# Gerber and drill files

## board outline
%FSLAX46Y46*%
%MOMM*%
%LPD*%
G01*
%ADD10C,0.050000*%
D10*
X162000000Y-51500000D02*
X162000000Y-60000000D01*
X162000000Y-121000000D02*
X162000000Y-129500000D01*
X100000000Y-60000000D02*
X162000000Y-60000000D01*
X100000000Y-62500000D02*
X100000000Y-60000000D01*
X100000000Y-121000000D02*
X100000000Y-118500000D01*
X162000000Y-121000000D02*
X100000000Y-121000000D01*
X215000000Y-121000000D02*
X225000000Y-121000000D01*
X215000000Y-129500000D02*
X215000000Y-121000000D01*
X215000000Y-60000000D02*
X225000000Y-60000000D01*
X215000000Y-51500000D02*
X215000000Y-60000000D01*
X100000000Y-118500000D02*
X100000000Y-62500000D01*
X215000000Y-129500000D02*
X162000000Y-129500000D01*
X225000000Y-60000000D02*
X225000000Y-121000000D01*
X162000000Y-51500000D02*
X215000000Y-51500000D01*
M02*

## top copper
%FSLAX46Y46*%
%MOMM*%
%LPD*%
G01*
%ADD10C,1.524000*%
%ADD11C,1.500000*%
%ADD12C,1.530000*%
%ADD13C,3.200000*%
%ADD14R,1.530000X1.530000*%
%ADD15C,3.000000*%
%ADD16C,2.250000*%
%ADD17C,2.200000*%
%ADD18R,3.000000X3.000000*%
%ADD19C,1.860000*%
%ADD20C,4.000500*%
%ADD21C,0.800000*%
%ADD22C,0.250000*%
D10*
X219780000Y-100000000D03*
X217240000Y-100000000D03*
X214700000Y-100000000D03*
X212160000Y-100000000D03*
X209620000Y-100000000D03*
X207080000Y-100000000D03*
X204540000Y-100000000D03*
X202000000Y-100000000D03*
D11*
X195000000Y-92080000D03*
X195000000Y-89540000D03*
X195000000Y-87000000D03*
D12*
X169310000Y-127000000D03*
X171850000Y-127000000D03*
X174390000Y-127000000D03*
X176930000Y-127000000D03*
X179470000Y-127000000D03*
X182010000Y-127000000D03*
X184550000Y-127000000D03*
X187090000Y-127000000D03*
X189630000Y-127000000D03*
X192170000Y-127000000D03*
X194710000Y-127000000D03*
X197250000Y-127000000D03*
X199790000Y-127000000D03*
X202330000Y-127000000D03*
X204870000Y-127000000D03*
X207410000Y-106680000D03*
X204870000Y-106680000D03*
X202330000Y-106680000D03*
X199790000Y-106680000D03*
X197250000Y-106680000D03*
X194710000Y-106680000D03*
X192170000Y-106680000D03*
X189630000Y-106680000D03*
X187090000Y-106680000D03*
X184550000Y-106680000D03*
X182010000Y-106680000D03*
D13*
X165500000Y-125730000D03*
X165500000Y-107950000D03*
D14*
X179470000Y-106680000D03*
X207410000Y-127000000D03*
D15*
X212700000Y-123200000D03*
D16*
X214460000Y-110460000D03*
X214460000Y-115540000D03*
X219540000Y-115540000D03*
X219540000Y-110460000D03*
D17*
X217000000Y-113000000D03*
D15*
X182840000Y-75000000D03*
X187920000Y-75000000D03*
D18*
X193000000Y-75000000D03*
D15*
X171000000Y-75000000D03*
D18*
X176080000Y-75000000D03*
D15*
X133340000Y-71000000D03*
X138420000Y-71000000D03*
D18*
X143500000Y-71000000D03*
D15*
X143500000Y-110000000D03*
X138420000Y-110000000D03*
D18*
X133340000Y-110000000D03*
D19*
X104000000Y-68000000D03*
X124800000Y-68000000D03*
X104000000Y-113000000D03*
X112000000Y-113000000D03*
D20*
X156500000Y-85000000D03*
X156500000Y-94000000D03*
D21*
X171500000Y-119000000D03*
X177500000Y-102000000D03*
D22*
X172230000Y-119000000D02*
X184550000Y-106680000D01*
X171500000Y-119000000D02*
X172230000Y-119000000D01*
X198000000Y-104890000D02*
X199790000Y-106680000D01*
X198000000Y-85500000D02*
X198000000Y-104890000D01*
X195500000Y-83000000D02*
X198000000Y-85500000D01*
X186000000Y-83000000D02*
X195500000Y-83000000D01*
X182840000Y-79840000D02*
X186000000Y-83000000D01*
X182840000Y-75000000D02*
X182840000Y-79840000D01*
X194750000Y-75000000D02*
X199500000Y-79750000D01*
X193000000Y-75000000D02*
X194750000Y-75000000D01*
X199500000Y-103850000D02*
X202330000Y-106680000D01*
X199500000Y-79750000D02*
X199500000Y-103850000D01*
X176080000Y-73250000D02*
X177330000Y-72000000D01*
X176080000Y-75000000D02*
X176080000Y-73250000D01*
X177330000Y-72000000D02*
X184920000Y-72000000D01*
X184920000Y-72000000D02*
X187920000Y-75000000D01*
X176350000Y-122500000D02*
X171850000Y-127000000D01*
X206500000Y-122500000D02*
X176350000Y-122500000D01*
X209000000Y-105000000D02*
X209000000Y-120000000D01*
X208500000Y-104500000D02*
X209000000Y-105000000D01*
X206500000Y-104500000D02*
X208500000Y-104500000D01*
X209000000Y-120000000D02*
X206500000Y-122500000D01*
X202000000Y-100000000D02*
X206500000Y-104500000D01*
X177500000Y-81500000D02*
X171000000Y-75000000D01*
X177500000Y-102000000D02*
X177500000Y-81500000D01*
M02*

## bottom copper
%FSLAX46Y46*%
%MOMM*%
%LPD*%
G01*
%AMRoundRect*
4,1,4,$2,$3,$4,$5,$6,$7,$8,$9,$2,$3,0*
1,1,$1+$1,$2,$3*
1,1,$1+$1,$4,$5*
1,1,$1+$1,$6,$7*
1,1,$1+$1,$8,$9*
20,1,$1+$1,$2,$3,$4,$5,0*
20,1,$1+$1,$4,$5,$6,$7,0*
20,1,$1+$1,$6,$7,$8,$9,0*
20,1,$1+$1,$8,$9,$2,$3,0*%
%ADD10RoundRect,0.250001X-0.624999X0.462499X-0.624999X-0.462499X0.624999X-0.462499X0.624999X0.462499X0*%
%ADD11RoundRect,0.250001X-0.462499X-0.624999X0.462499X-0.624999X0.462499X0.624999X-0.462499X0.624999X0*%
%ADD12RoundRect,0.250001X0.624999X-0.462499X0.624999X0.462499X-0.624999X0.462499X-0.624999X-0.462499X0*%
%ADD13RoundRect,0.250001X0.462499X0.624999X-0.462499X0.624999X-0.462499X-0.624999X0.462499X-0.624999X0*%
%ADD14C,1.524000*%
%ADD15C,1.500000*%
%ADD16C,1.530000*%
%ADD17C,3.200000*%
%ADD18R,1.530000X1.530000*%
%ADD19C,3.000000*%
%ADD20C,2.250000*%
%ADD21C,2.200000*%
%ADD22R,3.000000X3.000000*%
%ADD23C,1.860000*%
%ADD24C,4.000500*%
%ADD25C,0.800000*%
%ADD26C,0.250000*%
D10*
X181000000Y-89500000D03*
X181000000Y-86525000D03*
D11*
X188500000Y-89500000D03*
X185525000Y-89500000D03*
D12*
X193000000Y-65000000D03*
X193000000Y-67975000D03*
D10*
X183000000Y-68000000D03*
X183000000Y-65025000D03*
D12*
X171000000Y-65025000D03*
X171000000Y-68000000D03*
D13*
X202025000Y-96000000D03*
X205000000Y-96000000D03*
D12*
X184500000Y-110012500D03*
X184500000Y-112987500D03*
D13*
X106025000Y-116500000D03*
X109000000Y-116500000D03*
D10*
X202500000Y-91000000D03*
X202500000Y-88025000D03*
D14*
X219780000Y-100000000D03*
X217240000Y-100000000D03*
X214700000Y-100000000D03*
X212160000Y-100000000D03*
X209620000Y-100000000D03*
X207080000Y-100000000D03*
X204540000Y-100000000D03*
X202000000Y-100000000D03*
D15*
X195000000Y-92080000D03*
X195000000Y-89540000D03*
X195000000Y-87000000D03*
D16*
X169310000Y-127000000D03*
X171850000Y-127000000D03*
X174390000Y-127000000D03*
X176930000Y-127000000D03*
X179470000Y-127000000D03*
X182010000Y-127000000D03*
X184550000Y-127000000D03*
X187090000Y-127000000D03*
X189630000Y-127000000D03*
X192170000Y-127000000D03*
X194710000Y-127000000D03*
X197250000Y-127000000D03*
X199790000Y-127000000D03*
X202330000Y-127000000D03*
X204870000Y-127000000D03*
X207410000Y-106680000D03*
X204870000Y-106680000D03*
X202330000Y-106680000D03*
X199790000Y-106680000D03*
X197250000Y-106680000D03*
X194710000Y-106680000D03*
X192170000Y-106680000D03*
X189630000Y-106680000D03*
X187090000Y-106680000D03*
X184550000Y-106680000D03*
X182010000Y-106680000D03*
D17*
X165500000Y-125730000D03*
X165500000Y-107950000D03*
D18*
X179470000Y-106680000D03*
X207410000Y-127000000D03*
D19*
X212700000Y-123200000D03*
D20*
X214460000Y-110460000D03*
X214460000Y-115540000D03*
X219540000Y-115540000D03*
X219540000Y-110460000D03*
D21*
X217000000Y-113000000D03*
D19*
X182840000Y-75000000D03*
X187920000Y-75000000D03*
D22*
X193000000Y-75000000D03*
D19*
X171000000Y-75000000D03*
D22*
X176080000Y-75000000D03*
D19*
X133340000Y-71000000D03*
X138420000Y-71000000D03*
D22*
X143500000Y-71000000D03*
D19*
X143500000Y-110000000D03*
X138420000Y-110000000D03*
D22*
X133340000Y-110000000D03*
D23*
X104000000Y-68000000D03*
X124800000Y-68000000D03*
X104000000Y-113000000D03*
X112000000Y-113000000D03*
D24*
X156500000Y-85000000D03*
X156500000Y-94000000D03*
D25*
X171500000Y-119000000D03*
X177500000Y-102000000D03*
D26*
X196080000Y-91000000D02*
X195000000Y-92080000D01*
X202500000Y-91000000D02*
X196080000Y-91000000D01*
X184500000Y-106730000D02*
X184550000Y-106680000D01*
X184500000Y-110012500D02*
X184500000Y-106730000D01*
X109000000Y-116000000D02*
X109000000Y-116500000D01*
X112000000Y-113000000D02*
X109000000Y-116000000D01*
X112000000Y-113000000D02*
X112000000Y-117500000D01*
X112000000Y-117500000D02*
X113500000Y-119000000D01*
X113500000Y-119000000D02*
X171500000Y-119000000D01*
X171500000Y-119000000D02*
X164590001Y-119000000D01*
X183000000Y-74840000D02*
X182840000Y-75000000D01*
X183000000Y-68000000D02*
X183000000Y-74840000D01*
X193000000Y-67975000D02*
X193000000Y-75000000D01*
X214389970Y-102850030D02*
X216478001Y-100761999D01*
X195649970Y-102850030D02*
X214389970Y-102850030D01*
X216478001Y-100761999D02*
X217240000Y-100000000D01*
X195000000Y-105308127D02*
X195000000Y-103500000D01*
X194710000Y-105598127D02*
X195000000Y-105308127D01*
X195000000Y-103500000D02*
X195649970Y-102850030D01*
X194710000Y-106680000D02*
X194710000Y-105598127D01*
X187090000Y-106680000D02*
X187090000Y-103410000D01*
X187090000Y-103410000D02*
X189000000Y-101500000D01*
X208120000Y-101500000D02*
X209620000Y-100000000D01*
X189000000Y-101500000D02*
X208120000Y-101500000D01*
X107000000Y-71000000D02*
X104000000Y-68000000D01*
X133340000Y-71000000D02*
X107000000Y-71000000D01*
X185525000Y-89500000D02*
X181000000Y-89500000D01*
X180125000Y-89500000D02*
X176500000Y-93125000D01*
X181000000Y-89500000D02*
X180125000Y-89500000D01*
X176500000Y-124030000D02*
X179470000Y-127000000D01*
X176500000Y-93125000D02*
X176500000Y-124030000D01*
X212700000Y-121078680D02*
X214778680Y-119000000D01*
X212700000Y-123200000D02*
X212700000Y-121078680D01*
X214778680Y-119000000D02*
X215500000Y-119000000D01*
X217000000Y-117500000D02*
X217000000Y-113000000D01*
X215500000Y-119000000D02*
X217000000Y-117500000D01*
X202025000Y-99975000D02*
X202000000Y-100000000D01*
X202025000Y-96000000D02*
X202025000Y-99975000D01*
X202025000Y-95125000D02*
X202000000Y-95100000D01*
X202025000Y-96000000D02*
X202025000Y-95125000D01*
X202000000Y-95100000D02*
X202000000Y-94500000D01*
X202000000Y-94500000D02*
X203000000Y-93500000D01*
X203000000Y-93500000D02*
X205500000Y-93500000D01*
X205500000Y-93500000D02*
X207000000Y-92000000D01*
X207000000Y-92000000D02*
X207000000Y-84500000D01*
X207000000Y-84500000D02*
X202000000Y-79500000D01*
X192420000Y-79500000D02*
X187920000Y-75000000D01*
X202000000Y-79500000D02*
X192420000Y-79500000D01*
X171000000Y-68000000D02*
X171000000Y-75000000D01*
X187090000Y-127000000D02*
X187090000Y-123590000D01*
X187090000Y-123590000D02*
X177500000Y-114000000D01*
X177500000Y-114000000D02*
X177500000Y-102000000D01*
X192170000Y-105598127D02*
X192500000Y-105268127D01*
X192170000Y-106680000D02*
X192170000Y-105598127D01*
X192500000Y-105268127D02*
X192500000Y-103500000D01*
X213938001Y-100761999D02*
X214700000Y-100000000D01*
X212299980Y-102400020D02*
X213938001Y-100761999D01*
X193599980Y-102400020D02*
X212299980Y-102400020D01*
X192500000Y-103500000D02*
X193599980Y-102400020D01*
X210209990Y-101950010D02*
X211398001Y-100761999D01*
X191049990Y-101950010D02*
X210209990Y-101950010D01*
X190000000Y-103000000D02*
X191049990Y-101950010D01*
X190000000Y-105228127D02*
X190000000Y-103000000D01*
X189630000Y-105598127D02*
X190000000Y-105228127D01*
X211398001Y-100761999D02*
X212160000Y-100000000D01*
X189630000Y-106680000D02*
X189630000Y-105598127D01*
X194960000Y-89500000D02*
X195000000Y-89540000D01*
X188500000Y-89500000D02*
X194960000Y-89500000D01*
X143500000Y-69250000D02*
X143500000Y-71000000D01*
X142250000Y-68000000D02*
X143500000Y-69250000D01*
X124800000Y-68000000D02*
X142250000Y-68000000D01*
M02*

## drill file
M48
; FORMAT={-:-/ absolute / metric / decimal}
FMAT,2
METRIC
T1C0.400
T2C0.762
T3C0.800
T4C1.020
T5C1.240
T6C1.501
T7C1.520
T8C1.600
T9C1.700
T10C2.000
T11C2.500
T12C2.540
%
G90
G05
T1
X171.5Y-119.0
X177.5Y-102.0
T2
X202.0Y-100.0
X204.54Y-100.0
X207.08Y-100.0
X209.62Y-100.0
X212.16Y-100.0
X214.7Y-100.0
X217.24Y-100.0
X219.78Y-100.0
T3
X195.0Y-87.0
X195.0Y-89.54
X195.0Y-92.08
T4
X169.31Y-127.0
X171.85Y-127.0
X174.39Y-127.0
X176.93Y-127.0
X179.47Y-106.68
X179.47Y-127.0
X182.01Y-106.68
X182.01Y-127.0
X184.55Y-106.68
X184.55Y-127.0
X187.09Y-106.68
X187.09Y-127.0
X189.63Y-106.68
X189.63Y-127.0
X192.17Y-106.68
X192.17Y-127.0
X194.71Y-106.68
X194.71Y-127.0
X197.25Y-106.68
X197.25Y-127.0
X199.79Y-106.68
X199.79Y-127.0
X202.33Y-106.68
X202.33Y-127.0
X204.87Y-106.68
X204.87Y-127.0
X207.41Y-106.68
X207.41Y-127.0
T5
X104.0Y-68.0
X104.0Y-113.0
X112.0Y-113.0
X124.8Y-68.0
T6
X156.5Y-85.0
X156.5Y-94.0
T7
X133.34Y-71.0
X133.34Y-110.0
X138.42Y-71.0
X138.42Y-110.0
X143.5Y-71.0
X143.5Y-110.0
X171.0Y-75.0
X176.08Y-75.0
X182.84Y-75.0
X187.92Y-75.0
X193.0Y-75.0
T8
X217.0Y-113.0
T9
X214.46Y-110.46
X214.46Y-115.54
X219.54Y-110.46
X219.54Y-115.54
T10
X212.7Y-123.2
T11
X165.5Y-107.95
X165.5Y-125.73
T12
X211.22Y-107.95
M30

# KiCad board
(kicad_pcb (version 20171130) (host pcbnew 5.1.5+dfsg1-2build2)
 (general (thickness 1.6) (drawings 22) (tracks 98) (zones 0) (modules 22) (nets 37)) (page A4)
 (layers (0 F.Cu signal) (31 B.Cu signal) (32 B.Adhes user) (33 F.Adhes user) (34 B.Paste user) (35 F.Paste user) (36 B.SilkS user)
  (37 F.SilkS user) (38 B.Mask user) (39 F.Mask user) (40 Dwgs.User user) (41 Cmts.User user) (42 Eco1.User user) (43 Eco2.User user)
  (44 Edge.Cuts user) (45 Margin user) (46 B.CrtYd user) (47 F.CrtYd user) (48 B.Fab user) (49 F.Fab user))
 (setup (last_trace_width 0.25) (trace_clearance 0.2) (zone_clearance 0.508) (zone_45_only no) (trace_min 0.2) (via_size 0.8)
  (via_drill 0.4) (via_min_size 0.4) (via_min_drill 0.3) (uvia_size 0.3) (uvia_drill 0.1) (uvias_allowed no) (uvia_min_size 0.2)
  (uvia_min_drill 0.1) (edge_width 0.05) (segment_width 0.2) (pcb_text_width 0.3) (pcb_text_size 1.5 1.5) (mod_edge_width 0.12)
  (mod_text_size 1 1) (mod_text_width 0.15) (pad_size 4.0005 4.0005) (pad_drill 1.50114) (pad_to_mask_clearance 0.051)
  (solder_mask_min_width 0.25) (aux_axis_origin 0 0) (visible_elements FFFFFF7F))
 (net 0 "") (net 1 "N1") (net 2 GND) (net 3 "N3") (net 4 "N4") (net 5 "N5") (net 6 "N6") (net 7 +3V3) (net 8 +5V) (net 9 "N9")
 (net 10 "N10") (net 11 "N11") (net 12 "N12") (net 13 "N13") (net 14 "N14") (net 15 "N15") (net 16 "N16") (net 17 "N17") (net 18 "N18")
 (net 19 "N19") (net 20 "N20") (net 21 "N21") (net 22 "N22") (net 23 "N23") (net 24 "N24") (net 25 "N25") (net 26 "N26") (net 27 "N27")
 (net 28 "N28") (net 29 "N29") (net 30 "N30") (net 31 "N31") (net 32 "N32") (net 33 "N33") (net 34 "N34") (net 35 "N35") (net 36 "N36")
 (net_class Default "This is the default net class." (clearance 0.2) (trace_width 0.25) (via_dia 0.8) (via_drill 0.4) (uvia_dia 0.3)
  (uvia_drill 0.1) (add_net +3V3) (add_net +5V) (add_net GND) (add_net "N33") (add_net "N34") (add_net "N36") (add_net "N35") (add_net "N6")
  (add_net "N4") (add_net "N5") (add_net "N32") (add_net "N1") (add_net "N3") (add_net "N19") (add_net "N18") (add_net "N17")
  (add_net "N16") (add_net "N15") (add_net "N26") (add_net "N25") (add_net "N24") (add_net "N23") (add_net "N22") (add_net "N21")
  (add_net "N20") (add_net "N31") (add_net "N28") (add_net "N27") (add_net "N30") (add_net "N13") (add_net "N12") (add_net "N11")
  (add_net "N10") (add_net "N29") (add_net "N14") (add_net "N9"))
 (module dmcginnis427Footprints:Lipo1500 (layer F.Cu) (at 150.5 105.5 90)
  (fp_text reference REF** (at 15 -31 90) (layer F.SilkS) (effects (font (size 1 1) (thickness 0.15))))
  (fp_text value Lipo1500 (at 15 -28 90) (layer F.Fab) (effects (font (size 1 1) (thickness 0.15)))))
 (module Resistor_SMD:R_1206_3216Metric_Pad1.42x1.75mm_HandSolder (layer B.Cu) (at 181 88.0125 270)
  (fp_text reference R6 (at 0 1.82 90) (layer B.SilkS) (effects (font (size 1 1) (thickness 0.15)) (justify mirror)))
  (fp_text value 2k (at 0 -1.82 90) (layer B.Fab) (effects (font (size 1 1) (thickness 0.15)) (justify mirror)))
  (pad 2 smd roundrect (at 1.4875 0 270) (size 1.425 1.75) (layers B.Cu B.Paste B.Mask) (roundrect_rratio 0.175439) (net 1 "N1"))
  (pad 1 smd roundrect (at -1.4875 0 270) (size 1.425 1.75) (layers B.Cu B.Paste B.Mask) (roundrect_rratio 0.175439) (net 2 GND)))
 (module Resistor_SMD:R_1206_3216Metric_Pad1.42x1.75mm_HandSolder (layer B.Cu) (at 187.0125 89.5)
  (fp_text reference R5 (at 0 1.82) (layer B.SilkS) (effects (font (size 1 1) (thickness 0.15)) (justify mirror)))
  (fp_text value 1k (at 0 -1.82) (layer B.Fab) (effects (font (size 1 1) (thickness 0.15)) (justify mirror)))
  (pad 2 smd roundrect (at 1.4875 0) (size 1.425 1.75) (layers B.Cu B.Paste B.Mask) (roundrect_rratio 0.175439) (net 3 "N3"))
  (pad 1 smd roundrect (at -1.4875 0) (size 1.425 1.75) (layers B.Cu B.Paste B.Mask) (roundrect_rratio 0.175439) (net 1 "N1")))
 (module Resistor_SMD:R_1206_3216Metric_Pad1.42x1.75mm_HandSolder (layer B.Cu) (at 193 66.4875 90)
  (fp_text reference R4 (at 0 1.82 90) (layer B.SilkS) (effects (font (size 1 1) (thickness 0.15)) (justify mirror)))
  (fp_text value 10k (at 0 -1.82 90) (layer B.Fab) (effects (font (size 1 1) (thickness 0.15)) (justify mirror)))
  (pad 2 smd roundrect (at 1.4875 0 90) (size 1.425 1.75) (layers B.Cu B.Paste B.Mask) (roundrect_rratio 0.175439) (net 2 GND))
  (pad 1 smd roundrect (at -1.4875 0 90) (size 1.425 1.75) (layers B.Cu B.Paste B.Mask) (roundrect_rratio 0.175439) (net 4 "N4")))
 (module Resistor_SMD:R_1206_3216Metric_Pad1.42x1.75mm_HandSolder (layer B.Cu) (at 183 66.5125 270)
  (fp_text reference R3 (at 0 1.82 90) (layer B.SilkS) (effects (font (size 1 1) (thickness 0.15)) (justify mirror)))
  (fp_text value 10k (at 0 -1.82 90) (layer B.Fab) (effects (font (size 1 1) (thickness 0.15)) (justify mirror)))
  (pad 2 smd roundrect (at 1.4875 0 270) (size 1.425 1.75) (layers B.Cu B.Paste B.Mask) (roundrect_rratio 0.175439) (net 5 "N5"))
  (pad 1 smd roundrect (at -1.4875 0 270) (size 1.425 1.75) (layers B.Cu B.Paste B.Mask) (roundrect_rratio 0.175439) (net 2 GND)))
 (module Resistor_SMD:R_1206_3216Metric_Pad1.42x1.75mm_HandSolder (layer B.Cu) (at 171 66.5125 90)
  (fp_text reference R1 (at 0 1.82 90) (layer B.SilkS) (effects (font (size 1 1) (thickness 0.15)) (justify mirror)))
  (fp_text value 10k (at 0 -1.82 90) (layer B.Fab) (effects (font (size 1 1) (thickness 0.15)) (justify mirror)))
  (pad 2 smd roundrect (at 1.4875 0 90) (size 1.425 1.75) (layers B.Cu B.Paste B.Mask) (roundrect_rratio 0.175439) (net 2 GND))
  (pad 1 smd roundrect (at -1.4875 0 90) (size 1.425 1.75) (layers B.Cu B.Paste B.Mask) (roundrect_rratio 0.175439) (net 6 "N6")))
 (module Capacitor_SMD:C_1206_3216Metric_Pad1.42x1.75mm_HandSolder (layer B.Cu) (at 203.5125 96 180)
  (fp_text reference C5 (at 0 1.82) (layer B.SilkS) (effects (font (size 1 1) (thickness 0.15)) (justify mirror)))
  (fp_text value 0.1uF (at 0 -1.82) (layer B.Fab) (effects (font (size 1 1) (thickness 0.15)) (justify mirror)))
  (pad 2 smd roundrect (at 1.4875 0 180) (size 1.425 1.75) (layers B.Cu B.Paste B.Mask) (roundrect_rratio 0.175439) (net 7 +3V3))
  (pad 1 smd roundrect (at -1.4875 0 180) (size 1.425 1.75) (layers B.Cu B.Paste B.Mask) (roundrect_rratio 0.175439) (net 2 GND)))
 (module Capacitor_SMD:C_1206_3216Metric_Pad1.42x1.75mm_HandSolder (layer B.Cu) (at 184.5 111.5 90)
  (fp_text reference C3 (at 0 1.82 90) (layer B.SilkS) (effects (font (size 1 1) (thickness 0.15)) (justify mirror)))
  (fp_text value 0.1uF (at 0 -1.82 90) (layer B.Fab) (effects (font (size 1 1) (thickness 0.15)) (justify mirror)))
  (pad 2 smd roundrect (at 1.4875 0 90) (size 1.425 1.75) (layers B.Cu B.Paste B.Mask) (roundrect_rratio 0.175439) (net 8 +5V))
  (pad 1 smd roundrect (at -1.4875 0 90) (size 1.425 1.75) (layers B.Cu B.Paste B.Mask) (roundrect_rratio 0.175439) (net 2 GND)))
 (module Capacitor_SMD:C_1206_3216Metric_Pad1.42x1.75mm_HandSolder (layer B.Cu) (at 107.5125 116.5 180)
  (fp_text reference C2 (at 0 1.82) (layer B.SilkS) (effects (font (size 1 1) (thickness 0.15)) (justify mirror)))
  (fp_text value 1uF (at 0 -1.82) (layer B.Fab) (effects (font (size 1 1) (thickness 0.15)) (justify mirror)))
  (pad 2 smd roundrect (at 1.4875 0 180) (size 1.425 1.75) (layers B.Cu B.Paste B.Mask) (roundrect_rratio 0.175439) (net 2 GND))
  (pad 1 smd roundrect (at -1.4875 0 180) (size 1.425 1.75) (layers B.Cu B.Paste B.Mask) (roundrect_rratio 0.175439) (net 8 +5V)))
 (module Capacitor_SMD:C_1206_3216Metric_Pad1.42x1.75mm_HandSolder (layer B.Cu) (at 202.5 89.5125 270)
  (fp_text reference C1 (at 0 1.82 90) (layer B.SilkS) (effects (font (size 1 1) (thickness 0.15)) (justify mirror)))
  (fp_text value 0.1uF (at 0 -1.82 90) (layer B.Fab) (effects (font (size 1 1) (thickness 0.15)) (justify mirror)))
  (pad 2 smd roundrect (at 1.4875 0 270) (size 1.425 1.75) (layers B.Cu B.Paste B.Mask) (roundrect_rratio 0.175439) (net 8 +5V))
  (pad 1 smd roundrect (at -1.4875 0 270) (size 1.425 1.75) (layers B.Cu B.Paste B.Mask) (roundrect_rratio 0.175439) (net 2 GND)))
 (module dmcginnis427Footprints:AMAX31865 (layer F.Cu) (at 202 100)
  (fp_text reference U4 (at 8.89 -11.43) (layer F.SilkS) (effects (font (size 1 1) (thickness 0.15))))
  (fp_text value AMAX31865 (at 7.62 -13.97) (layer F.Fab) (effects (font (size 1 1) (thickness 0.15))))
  (pad 8 thru_hole circle (at 17.78 0) (size 1.524 1.524) (drill 0.762) (layers *.Cu *.Mask) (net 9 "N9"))
  (pad 7 thru_hole circle (at 15.24 0) (size 1.524 1.524) (drill 0.762) (layers *.Cu *.Mask) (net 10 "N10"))
  (pad 6 thru_hole circle (at 12.7 0) (size 1.524 1.524) (drill 0.762) (layers *.Cu *.Mask) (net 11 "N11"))
  (pad 5 thru_hole circle (at 10.16 0) (size 1.524 1.524) (drill 0.762) (layers *.Cu *.Mask) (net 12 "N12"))
  (pad 4 thru_hole circle (at 7.62 0) (size 1.524 1.524) (drill 0.762) (layers *.Cu *.Mask) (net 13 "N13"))
  (pad 3 thru_hole circle (at 5.08 0) (size 1.524 1.524) (drill 0.762) (layers *.Cu *.Mask) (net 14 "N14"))
  (pad 2 thru_hole circle (at 2.54 0) (size 1.524 1.524) (drill 0.762) (layers *.Cu *.Mask) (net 2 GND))
  (pad 1 thru_hole circle (at 0 0) (size 1.524 1.524) (drill 0.762) (layers *.Cu *.Mask) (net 7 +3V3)))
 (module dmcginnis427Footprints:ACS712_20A (layer F.Cu) (at 195 89.54 270)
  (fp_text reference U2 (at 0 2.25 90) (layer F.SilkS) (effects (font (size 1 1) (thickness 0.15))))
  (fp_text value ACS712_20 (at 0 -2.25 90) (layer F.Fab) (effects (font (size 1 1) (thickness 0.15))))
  (pad 3 thru_hole circle (at 2.54 0 270) (size 1.5 1.5) (drill 0.8) (layers *.Cu *.Mask) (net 8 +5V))
  (pad 2 thru_hole circle (at 0 0 270) (size 1.5 1.5) (drill 0.8) (layers *.Cu *.Mask) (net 3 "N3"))
  (pad 1 thru_hole circle (at -2.54 0 270) (size 1.5 1.5) (drill 0.8) (layers *.Cu *.Mask) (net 2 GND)))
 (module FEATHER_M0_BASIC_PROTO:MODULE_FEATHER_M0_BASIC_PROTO (layer F.Cu) (at 188.36 116.84)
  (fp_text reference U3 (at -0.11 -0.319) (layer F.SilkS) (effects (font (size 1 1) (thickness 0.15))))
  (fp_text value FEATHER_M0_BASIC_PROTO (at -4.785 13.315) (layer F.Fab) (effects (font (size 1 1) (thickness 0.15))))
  (pad P1_16 thru_hole circle (at -19.05 10.16) (size 1.53 1.53) (drill 1.02) (layers *.Cu *.Mask) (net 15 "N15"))
  (pad P1_15 thru_hole circle (at -16.51 10.16) (size 1.53 1.53) (drill 1.02) (layers *.Cu *.Mask) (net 7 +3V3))
  (pad P1_14 thru_hole circle (at -13.97 10.16) (size 1.53 1.53) (drill 1.02) (layers *.Cu *.Mask) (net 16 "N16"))
  (pad P1_13 thru_hole circle (at -11.43 10.16) (size 1.53 1.53) (drill 1.02) (layers *.Cu *.Mask) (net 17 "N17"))
  (pad P1_12 thru_hole circle (at -8.89 10.16) (size 1.53 1.53) (drill 1.02) (layers *.Cu *.Mask) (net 1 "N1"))
  (pad P1_11 thru_hole circle (at -6.35 10.16) (size 1.53 1.53) (drill 1.02) (layers *.Cu *.Mask) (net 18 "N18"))
  (pad P1_10 thru_hole circle (at -3.81 10.16) (size 1.53 1.53) (drill 1.02) (layers *.Cu *.Mask) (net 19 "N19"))
  (pad P1_9 thru_hole circle (at -1.27 10.16) (size 1.53 1.53) (drill 1.02) (layers *.Cu *.Mask) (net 6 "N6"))
  (pad P1_8 thru_hole circle (at 1.27 10.16) (size 1.53 1.53) (drill 1.02) (layers *.Cu *.Mask) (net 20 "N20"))
  (pad P1_7 thru_hole circle (at 3.81 10.16) (size 1.53 1.53) (drill 1.02) (layers *.Cu *.Mask) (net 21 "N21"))
  (pad P1_6 thru_hole circle (at 6.35 10.16) (size 1.53 1.53) (drill 1.02) (layers *.Cu *.Mask) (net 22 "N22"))
  (pad P1_5 thru_hole circle (at 8.89 10.16) (size 1.53 1.53) (drill 1.02) (layers *.Cu *.Mask) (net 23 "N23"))
  (pad P1_4 thru_hole circle (at 11.43 10.16) (size 1.53 1.53) (drill 1.02) (layers *.Cu *.Mask) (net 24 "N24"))
  (pad P1_3 thru_hole circle (at 13.97 10.16) (size 1.53 1.53) (drill 1.02) (layers *.Cu *.Mask) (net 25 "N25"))
  (pad P1_2 thru_hole circle (at 16.51 10.16) (size 1.53 1.53) (drill 1.02) (layers *.Cu *.Mask) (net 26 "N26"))
  (pad P2_12 thru_hole circle (at 19.05 -10.16) (size 1.53 1.53) (drill 1.02) (layers *.Cu *.Mask) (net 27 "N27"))
  (pad P2_11 thru_hole circle (at 16.51 -10.16) (size 1.53 1.53) (drill 1.02) (layers *.Cu *.Mask) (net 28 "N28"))
  (pad P2_10 thru_hole circle (at 13.97 -10.16) (size 1.53 1.53) (drill 1.02) (layers *.Cu *.Mask) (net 4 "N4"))
  (pad P2_9 thru_hole circle (at 11.43 -10.16) (size 1.53 1.53) (drill 1.02) (layers *.Cu *.Mask) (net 5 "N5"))
  (pad P2_8 thru_hole circle (at 8.89 -10.16) (size 1.53 1.53) (drill 1.02) (layers *.Cu *.Mask) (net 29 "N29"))
  (pad P2_7 thru_hole circle (at 6.35 -10.16) (size 1.53 1.53) (drill 1.02) (layers *.Cu *.Mask) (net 10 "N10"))
  (pad P2_6 thru_hole circle (at 3.81 -10.16) (size 1.53 1.53) (drill 1.02) (layers *.Cu *.Mask) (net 11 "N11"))
  (pad P2_5 thru_hole circle (at 1.27 -10.16) (size 1.53 1.53) (drill 1.02) (layers *.Cu *.Mask) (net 12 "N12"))
  (pad P2_4 thru_hole circle (at -1.27 -10.16) (size 1.53 1.53) (drill 1.02) (layers *.Cu *.Mask) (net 13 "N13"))
  (pad P2_3 thru_hole circle (at -3.81 -10.16) (size 1.53 1.53) (drill 1.02) (layers *.Cu *.Mask) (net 8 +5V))
  (pad P2_2 thru_hole circle (at -6.35 -10.16) (size 1.53 1.53) (drill 1.02) (layers *.Cu *.Mask) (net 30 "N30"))
  (pad None np_thru_hole circle (at 22.86 -8.89) (size 2.54 2.54) (drill 2.54) (layers *.Cu *.Mask))
  (pad P$2 thru_hole circle (at -22.86 8.89) (size 3.2 3.2) (drill 2.5) (layers *.Cu *.Mask))
  (pad P$1 thru_hole circle (at -22.86 -8.89) (size 3.2 3.2) (drill 2.5) (layers *.Cu *.Mask))
  (pad P2_1 thru_hole rect (at -8.89 -10.16) (size 1.53 1.53) (drill 1.02) (layers *.Cu *.Mask) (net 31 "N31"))
  (pad P1_1 thru_hole rect (at 19.05 10.16) (size 1.53 1.53) (drill 1.02) (layers *.Cu *.Mask) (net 2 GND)))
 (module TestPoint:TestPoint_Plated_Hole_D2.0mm (layer B.Cu) (at 212.7 123.2)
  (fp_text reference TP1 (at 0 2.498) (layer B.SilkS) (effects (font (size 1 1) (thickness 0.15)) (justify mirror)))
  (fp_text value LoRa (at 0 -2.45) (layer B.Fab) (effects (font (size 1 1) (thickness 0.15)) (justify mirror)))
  (pad 1 thru_hole circle (at 0 0) (size 3 3) (drill 2) (layers *.Cu *.Mask) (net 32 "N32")))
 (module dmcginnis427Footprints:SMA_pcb (layer B.Cu) (at 217 113)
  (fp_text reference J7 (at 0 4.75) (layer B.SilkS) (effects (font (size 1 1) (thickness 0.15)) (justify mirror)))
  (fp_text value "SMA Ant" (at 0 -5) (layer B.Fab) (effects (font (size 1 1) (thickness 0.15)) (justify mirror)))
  (pad 2 thru_hole circle (at -2.54 -2.54) (size 2.25 2.25) (drill 1.7) (layers *.Cu *.Mask) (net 2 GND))
  (pad 2 thru_hole circle (at -2.54 2.54) (size 2.25 2.25) (drill 1.7) (layers *.Cu *.Mask) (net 2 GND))
  (pad 2 thru_hole circle (at 2.54 2.54) (size 2.25 2.25) (drill 1.7) (layers *.Cu *.Mask) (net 2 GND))
  (pad 2 thru_hole circle (at 2.54 -2.54) (size 2.25 2.25) (drill 1.7) (layers *.Cu *.Mask) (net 2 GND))
  (pad 1 thru_hole circle (at 0 0) (size 2.2 2.2) (drill 1.6) (layers *.Cu *.Mask) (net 32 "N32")))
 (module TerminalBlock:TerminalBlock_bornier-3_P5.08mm (layer F.Cu) (at 193 75 180)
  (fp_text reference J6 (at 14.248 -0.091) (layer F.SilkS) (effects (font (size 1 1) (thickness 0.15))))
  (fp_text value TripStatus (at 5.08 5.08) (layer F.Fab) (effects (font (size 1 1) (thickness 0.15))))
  (pad 3 thru_hole circle (at 10.16 0 180) (size 3 3) (drill 1.52) (layers *.Cu *.Mask) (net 5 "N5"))
  (pad 2 thru_hole circle (at 5.08 0 180) (size 3 3) (drill 1.52) (layers *.Cu *.Mask) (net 7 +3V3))
  (pad 1 thru_hole rect (at 0 0 180) (size 3 3) (drill 1.52) (layers *.Cu *.Mask) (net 4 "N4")))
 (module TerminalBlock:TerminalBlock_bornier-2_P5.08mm (layer F.Cu) (at 176.08 75 180)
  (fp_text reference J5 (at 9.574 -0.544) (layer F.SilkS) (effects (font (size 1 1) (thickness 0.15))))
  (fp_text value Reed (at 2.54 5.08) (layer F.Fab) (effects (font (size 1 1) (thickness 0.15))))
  (pad 2 thru_hole circle (at 5.08 0 180) (size 3 3) (drill 1.52) (layers *.Cu *.Mask) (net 6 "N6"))
  (pad 1 thru_hole rect (at 0 0 180) (size 3 3) (drill 1.52) (layers *.Cu *.Mask) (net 7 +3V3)))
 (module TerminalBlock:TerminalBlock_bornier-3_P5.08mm (layer F.Cu) (at 143.5 71 180)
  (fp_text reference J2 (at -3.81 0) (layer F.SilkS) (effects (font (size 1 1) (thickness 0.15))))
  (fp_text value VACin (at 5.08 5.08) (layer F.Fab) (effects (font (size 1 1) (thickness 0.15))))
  (pad 3 thru_hole circle (at 10.16 0 180) (size 3 3) (drill 1.52) (layers *.Cu *.Mask) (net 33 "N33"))
  (pad 2 thru_hole circle (at 5.08 0 180) (size 3 3) (drill 1.52) (layers *.Cu *.Mask) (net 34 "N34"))
  (pad 1 thru_hole rect (at 0 0 180) (size 3 3) (drill 1.52) (layers *.Cu *.Mask) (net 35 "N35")))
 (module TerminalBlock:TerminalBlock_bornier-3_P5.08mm (layer F.Cu) (at 133.34 110)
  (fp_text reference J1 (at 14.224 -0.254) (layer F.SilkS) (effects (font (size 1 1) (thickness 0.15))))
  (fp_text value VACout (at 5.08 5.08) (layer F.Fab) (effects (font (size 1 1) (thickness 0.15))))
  (pad 3 thru_hole circle (at 10.16 0) (size 3 3) (drill 1.52) (layers *.Cu *.Mask) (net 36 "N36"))
  (pad 2 thru_hole circle (at 5.08 0) (size 3 3) (drill 1.52) (layers *.Cu *.Mask) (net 34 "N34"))
  (pad 1 thru_hole rect (at 0 0) (size 3 3) (drill 1.52) (layers *.Cu *.Mask) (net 33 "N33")))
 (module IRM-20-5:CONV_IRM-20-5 (layer F.Cu) (at 114.4 90.8 270)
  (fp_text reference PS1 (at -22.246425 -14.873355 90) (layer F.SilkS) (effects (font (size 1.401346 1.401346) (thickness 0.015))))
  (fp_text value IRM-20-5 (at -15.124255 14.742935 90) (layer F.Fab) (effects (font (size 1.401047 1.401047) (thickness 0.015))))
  (pad 2 thru_hole circle (at -22.8 10.4 270) (size 1.86 1.86) (drill 1.24) (layers *.Cu *.Mask) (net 33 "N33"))
  (pad 1 thru_hole circle (at -22.8 -10.4 270) (size 1.86 1.86) (drill 1.24) (layers *.Cu *.Mask) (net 35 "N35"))
  (pad 3 thru_hole circle (at 22.2 10.4 270) (size 1.86 1.86) (drill 1.24) (layers *.Cu *.Mask) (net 2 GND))
  (pad 4 thru_hole circle (at 22.2 2.4 270) (size 1.86 1.86) (drill 1.24) (layers *.Cu *.Mask) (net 8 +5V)))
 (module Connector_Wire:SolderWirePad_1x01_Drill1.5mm (layer F.Cu) (at 156.5 85)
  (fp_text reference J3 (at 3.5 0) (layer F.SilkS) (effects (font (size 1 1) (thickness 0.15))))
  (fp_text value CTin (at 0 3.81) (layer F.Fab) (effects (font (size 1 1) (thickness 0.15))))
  (pad 1 thru_hole circle (at 0 0) (size 4.0005 4.0005) (drill 1.50114) (layers *.Mask B.Cu) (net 35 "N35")))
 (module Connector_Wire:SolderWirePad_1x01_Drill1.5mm (layer F.Cu) (at 156.5 94)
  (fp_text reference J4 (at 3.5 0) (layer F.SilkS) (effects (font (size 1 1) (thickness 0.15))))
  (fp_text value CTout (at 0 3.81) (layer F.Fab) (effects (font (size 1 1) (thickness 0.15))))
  (pad 1 thru_hole circle (at 0 0) (size 4.0005 4.0005) (drill 1.50114) (layers *.Mask B.Cu) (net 36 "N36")))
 (gr_line (start 162 51.5) (end 162 60) (layer Edge.Cuts) (width 0.05))
 (gr_line (start 162 121) (end 162 129.5) (layer Edge.Cuts) (width 0.05))
 (gr_line (start 100 60) (end 162 60) (layer Edge.Cuts) (width 0.05))
 (gr_line (start 100 62.5) (end 100 60) (layer Edge.Cuts) (width 0.05))
 (gr_line (start 100 121) (end 100 118.5) (layer Edge.Cuts) (width 0.05))
 (gr_line (start 162 121) (end 100 121) (layer Edge.Cuts) (width 0.05))
 (gr_line (start 215 121) (end 225 121) (layer Edge.Cuts) (width 0.05))
 (gr_line (start 215 129.5) (end 215 121) (layer Edge.Cuts) (width 0.05))
 (gr_line (start 215 60) (end 225 60) (layer Edge.Cuts) (width 0.05))
 (gr_line (start 215 51.5) (end 215 60) (layer Edge.Cuts) (width 0.05))
 (gr_line (start 100 118.5) (end 100 62.5) (layer Edge.Cuts) (width 0.05))
 (gr_line (start 215 129.5) (end 162 129.5) (layer Edge.Cuts) (width 0.05))
 (gr_line (start 225 60) (end 225 121) (layer Edge.Cuts) (width 0.05))
 (gr_line (start 162 51.5) (end 215 51.5) (layer Edge.Cuts) (width 0.05))
 (segment (start 196.08 91) (end 195 92.08) (width 0.25) (layer B.Cu) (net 8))
 (segment (start 202.5 91) (end 196.08 91) (width 0.25) (layer B.Cu) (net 8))
 (segment (start 184.5 106.73) (end 184.55 106.68) (width 0.25) (layer B.Cu) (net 8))
 (segment (start 184.5 110.0125) (end 184.5 106.73) (width 0.25) (layer B.Cu) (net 8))
 (segment (start 109 116) (end 109 116.5) (width 0.25) (layer B.Cu) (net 8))
 (segment (start 112 113) (end 109 116) (width 0.25) (layer B.Cu) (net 8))
 (segment (start 112 113) (end 112 117.5) (width 0.25) (layer B.Cu) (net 8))
 (segment (start 112 117.5) (end 113.5 119) (width 0.25) (layer B.Cu) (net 8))
 (segment (start 113.5 119) (end 171.5 119) (width 0.25) (layer B.Cu) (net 8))
 (via (at 171.5 119) (size 0.8) (drill 0.4) (layers F.Cu B.Cu) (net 8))
 (segment (start 171.5 119) (end 164.590001 119) (width 0.25) (layer B.Cu) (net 8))
 (segment (start 172.23 119) (end 184.55 106.68) (width 0.25) (layer F.Cu) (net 8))
 (segment (start 171.5 119) (end 172.23 119) (width 0.25) (layer F.Cu) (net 8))
 (segment (start 183 74.84) (end 182.84 75) (width 0.25) (layer B.Cu) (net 5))
 (segment (start 183 68) (end 183 74.84) (width 0.25) (layer B.Cu) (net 5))
 (segment (start 198 104.89) (end 199.79 106.68) (width 0.25) (layer F.Cu) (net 5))
 (segment (start 198 85.5) (end 198 104.89) (width 0.25) (layer F.Cu) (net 5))
 (segment (start 195.5 83) (end 198 85.5) (width 0.25) (layer F.Cu) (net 5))
 (segment (start 186 83) (end 195.5 83) (width 0.25) (layer F.Cu) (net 5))
 (segment (start 182.84 79.84) (end 186 83) (width 0.25) (layer F.Cu) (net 5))
 (segment (start 182.84 75) (end 182.84 79.84) (width 0.25) (layer F.Cu) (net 5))
 (segment (start 193 67.975) (end 193 75) (width 0.25) (layer B.Cu) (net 4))
 (segment (start 194.75 75) (end 199.5 79.75) (width 0.25) (layer F.Cu) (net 4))
 (segment (start 193 75) (end 194.75 75) (width 0.25) (layer F.Cu) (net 4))
 (segment (start 199.5 103.85) (end 202.33 106.68) (width 0.25) (layer F.Cu) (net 4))
 (segment (start 199.5 79.75) (end 199.5 103.85) (width 0.25) (layer F.Cu) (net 4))
 (segment (start 214.38997 102.85003) (end 216.478001 100.761999) (width 0.25) (layer B.Cu) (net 10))
 (segment (start 195.64997 102.85003) (end 214.38997 102.85003) (width 0.25) (layer B.Cu) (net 10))
 (segment (start 216.478001 100.761999) (end 217.24 100) (width 0.25) (layer B.Cu) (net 10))
 (segment (start 195 105.308127) (end 195 103.5) (width 0.25) (layer B.Cu) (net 10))
 (segment (start 194.71 105.598127) (end 195 105.308127) (width 0.25) (layer B.Cu) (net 10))
 (segment (start 195 103.5) (end 195.64997 102.85003) (width 0.25) (layer B.Cu) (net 10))
 (segment (start 194.71 106.68) (end 194.71 105.598127) (width 0.25) (layer B.Cu) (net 10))
 (segment (start 187.09 106.68) (end 187.09 103.41) (width 0.25) (layer B.Cu) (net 13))
 (segment (start 187.09 103.41) (end 189 101.5) (width 0.25) (layer B.Cu) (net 13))
 (segment (start 208.12 101.5) (end 209.62 100) (width 0.25) (layer B.Cu) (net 13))
 (segment (start 189 101.5) (end 208.12 101.5) (width 0.25) (layer B.Cu) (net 13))
 (segment (start 107 71) (end 104 68) (width 0.25) (layer B.Cu) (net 33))
 (segment (start 133.34 71) (end 107 71) (width 0.25) (layer B.Cu) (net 33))
 (segment (start 185.525 89.5) (end 181 89.5) (width 0.25) (layer B.Cu) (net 1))
 (segment (start 180.125 89.5) (end 176.5 93.125) (width 0.25) (layer B.Cu) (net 1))
 (segment (start 181 89.5) (end 180.125 89.5) (width 0.25) (layer B.Cu) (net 1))
 (segment (start 176.5 124.03) (end 179.47 127) (width 0.25) (layer B.Cu) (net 1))
 (segment (start 176.5 93.125) (end 176.5 124.03) (width 0.25) (layer B.Cu) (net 1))
 (segment (start 212.7 121.07868) (end 214.77868 119) (width 0.25) (layer B.Cu) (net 32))
 (segment (start 212.7 123.2) (end 212.7 121.07868) (width 0.25) (layer B.Cu) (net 32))
 (segment (start 214.77868 119) (end 215.5 119) (width 0.25) (layer B.Cu) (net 32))
 (segment (start 217 117.5) (end 217 113) (width 0.25) (layer B.Cu) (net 32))
 (segment (start 215.5 119) (end 217 117.5) (width 0.25) (layer B.Cu) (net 32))
 (segment (start 202.025 99.975) (end 202 100) (width 0.25) (layer B.Cu) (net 7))
 (segment (start 202.025 96) (end 202.025 99.975) (width 0.25) (layer B.Cu) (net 7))
 (segment (start 176.08 73.25) (end 177.33 72) (width 0.25) (layer F.Cu) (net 7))
 (segment (start 176.08 75) (end 176.08 73.25) (width 0.25) (layer F.Cu) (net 7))
 (segment (start 177.33 72) (end 184.92 72) (width 0.25) (layer F.Cu) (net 7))
 (segment (start 184.92 72) (end 187.92 75) (width 0.25) (layer F.Cu) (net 7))
 (segment (start 176.35 122.5) (end 171.85 127) (width 0.25) (layer F.Cu) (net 7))
 (segment (start 206.5 122.5) (end 176.35 122.5) (width 0.25) (layer F.Cu) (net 7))
 (segment (start 209 105) (end 209 120) (width 0.25) (layer F.Cu) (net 7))
 (segment (start 208.5 104.5) (end 209 105) (width 0.25) (layer F.Cu) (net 7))
 (segment (start 206.5 104.5) (end 208.5 104.5) (width 0.25) (layer F.Cu) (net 7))
 (segment (start 209 120) (end 206.5 122.5) (width 0.25) (layer F.Cu) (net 7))
 (segment (start 202 100) (end 206.5 104.5) (width 0.25) (layer F.Cu) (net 7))
 (segment (start 202.025 95.125) (end 202 95.1) (width 0.25) (layer B.Cu) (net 7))
 (segment (start 202.025 96) (end 202.025 95.125) (width 0.25) (layer B.Cu) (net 7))
 (segment (start 202 95.1) (end 202 94.5) (width 0.25) (layer B.Cu) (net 7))
 (segment (start 202 94.5) (end 203 93.5) (width 0.25) (layer B.Cu) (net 7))
 (segment (start 203 93.5) (end 205.5 93.5) (width 0.25) (layer B.Cu) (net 7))
 (segment (start 205.5 93.5) (end 207 92) (width 0.25) (layer B.Cu) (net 7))
 (segment (start 207 92) (end 207 84.5) (width 0.25) (layer B.Cu) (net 7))
 (segment (start 207 84.5) (end 202 79.5) (width 0.25) (layer B.Cu) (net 7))
 (segment (start 192.42 79.5) (end 187.92 75) (width 0.25) (layer B.Cu) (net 7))
 (segment (start 202 79.5) (end 192.42 79.5) (width 0.25) (layer B.Cu) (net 7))
 (segment (start 171 68) (end 171 75) (width 0.25) (layer B.Cu) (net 6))
 (segment (start 187.09 127) (end 187.09 123.59) (width 0.25) (layer B.Cu) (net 6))
 (segment (start 187.09 123.59) (end 177.5 114) (width 0.25) (layer B.Cu) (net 6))
 (segment (start 177.5 114) (end 177.5 102) (width 0.25) (layer B.Cu) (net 6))
 (via (at 177.5 102) (size 0.8) (drill 0.4) (layers F.Cu B.Cu) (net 6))
 (segment (start 177.5 81.5) (end 171 75) (width 0.25) (layer F.Cu) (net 6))
 (segment (start 177.5 102) (end 177.5 81.5) (width 0.25) (layer F.Cu) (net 6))
 (segment (start 192.17 105.598127) (end 192.5 105.268127) (width 0.25) (layer B.Cu) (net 11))
 (segment (start 192.17 106.68) (end 192.17 105.598127) (width 0.25) (layer B.Cu) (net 11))
 (segment (start 192.5 105.268127) (end 192.5 103.5) (width 0.25) (layer B.Cu) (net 11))
 (segment (start 213.938001 100.761999) (end 214.7 100) (width 0.25) (layer B.Cu) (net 11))
 (segment (start 212.29998 102.40002) (end 213.938001 100.761999) (width 0.25) (layer B.Cu) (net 11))
 (segment (start 193.59998 102.40002) (end 212.29998 102.40002) (width 0.25) (layer B.Cu) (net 11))
 (segment (start 192.5 103.5) (end 193.59998 102.40002) (width 0.25) (layer B.Cu) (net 11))
 (segment (start 210.20999 101.95001) (end 211.398001 100.761999) (width 0.25) (layer B.Cu) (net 12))
 (segment (start 191.04999 101.95001) (end 210.20999 101.95001) (width 0.25) (layer B.Cu) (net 12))
 (segment (start 190 103) (end 191.04999 101.95001) (width 0.25) (layer B.Cu) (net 12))
 (segment (start 190 105.228127) (end 190 103) (width 0.25) (layer B.Cu) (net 12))
 (segment (start 189.63 105.598127) (end 190 105.228127) (width 0.25) (layer B.Cu) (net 12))
 (segment (start 211.398001 100.761999) (end 212.16 100) (width 0.25) (layer B.Cu) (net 12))
 (segment (start 189.63 106.68) (end 189.63 105.598127) (width 0.25) (layer B.Cu) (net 12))
 (segment (start 194.96 89.5) (end 195 89.54) (width 0.25) (layer B.Cu) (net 3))
 (segment (start 188.5 89.5) (end 194.96 89.5) (width 0.25) (layer B.Cu) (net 3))
 (segment (start 143.5 69.25) (end 143.5 71) (width 0.25) (layer B.Cu) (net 35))
 (segment (start 142.25 68) (end 143.5 69.25) (width 0.25) (layer B.Cu) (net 35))
 (segment (start 124.8 68) (end 142.25 68) (width 0.25) (layer B.Cu) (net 35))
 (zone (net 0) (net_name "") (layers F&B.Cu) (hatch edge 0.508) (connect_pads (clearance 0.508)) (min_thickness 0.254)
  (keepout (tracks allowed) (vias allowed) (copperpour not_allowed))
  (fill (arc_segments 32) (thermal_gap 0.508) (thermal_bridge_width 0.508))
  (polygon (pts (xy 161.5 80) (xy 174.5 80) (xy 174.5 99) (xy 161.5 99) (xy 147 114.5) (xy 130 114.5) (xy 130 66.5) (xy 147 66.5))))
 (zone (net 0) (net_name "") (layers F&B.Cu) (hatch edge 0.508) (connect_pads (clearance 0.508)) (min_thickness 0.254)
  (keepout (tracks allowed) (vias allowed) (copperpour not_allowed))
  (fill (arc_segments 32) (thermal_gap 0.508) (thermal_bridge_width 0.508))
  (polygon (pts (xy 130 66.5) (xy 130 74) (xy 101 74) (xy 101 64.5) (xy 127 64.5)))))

